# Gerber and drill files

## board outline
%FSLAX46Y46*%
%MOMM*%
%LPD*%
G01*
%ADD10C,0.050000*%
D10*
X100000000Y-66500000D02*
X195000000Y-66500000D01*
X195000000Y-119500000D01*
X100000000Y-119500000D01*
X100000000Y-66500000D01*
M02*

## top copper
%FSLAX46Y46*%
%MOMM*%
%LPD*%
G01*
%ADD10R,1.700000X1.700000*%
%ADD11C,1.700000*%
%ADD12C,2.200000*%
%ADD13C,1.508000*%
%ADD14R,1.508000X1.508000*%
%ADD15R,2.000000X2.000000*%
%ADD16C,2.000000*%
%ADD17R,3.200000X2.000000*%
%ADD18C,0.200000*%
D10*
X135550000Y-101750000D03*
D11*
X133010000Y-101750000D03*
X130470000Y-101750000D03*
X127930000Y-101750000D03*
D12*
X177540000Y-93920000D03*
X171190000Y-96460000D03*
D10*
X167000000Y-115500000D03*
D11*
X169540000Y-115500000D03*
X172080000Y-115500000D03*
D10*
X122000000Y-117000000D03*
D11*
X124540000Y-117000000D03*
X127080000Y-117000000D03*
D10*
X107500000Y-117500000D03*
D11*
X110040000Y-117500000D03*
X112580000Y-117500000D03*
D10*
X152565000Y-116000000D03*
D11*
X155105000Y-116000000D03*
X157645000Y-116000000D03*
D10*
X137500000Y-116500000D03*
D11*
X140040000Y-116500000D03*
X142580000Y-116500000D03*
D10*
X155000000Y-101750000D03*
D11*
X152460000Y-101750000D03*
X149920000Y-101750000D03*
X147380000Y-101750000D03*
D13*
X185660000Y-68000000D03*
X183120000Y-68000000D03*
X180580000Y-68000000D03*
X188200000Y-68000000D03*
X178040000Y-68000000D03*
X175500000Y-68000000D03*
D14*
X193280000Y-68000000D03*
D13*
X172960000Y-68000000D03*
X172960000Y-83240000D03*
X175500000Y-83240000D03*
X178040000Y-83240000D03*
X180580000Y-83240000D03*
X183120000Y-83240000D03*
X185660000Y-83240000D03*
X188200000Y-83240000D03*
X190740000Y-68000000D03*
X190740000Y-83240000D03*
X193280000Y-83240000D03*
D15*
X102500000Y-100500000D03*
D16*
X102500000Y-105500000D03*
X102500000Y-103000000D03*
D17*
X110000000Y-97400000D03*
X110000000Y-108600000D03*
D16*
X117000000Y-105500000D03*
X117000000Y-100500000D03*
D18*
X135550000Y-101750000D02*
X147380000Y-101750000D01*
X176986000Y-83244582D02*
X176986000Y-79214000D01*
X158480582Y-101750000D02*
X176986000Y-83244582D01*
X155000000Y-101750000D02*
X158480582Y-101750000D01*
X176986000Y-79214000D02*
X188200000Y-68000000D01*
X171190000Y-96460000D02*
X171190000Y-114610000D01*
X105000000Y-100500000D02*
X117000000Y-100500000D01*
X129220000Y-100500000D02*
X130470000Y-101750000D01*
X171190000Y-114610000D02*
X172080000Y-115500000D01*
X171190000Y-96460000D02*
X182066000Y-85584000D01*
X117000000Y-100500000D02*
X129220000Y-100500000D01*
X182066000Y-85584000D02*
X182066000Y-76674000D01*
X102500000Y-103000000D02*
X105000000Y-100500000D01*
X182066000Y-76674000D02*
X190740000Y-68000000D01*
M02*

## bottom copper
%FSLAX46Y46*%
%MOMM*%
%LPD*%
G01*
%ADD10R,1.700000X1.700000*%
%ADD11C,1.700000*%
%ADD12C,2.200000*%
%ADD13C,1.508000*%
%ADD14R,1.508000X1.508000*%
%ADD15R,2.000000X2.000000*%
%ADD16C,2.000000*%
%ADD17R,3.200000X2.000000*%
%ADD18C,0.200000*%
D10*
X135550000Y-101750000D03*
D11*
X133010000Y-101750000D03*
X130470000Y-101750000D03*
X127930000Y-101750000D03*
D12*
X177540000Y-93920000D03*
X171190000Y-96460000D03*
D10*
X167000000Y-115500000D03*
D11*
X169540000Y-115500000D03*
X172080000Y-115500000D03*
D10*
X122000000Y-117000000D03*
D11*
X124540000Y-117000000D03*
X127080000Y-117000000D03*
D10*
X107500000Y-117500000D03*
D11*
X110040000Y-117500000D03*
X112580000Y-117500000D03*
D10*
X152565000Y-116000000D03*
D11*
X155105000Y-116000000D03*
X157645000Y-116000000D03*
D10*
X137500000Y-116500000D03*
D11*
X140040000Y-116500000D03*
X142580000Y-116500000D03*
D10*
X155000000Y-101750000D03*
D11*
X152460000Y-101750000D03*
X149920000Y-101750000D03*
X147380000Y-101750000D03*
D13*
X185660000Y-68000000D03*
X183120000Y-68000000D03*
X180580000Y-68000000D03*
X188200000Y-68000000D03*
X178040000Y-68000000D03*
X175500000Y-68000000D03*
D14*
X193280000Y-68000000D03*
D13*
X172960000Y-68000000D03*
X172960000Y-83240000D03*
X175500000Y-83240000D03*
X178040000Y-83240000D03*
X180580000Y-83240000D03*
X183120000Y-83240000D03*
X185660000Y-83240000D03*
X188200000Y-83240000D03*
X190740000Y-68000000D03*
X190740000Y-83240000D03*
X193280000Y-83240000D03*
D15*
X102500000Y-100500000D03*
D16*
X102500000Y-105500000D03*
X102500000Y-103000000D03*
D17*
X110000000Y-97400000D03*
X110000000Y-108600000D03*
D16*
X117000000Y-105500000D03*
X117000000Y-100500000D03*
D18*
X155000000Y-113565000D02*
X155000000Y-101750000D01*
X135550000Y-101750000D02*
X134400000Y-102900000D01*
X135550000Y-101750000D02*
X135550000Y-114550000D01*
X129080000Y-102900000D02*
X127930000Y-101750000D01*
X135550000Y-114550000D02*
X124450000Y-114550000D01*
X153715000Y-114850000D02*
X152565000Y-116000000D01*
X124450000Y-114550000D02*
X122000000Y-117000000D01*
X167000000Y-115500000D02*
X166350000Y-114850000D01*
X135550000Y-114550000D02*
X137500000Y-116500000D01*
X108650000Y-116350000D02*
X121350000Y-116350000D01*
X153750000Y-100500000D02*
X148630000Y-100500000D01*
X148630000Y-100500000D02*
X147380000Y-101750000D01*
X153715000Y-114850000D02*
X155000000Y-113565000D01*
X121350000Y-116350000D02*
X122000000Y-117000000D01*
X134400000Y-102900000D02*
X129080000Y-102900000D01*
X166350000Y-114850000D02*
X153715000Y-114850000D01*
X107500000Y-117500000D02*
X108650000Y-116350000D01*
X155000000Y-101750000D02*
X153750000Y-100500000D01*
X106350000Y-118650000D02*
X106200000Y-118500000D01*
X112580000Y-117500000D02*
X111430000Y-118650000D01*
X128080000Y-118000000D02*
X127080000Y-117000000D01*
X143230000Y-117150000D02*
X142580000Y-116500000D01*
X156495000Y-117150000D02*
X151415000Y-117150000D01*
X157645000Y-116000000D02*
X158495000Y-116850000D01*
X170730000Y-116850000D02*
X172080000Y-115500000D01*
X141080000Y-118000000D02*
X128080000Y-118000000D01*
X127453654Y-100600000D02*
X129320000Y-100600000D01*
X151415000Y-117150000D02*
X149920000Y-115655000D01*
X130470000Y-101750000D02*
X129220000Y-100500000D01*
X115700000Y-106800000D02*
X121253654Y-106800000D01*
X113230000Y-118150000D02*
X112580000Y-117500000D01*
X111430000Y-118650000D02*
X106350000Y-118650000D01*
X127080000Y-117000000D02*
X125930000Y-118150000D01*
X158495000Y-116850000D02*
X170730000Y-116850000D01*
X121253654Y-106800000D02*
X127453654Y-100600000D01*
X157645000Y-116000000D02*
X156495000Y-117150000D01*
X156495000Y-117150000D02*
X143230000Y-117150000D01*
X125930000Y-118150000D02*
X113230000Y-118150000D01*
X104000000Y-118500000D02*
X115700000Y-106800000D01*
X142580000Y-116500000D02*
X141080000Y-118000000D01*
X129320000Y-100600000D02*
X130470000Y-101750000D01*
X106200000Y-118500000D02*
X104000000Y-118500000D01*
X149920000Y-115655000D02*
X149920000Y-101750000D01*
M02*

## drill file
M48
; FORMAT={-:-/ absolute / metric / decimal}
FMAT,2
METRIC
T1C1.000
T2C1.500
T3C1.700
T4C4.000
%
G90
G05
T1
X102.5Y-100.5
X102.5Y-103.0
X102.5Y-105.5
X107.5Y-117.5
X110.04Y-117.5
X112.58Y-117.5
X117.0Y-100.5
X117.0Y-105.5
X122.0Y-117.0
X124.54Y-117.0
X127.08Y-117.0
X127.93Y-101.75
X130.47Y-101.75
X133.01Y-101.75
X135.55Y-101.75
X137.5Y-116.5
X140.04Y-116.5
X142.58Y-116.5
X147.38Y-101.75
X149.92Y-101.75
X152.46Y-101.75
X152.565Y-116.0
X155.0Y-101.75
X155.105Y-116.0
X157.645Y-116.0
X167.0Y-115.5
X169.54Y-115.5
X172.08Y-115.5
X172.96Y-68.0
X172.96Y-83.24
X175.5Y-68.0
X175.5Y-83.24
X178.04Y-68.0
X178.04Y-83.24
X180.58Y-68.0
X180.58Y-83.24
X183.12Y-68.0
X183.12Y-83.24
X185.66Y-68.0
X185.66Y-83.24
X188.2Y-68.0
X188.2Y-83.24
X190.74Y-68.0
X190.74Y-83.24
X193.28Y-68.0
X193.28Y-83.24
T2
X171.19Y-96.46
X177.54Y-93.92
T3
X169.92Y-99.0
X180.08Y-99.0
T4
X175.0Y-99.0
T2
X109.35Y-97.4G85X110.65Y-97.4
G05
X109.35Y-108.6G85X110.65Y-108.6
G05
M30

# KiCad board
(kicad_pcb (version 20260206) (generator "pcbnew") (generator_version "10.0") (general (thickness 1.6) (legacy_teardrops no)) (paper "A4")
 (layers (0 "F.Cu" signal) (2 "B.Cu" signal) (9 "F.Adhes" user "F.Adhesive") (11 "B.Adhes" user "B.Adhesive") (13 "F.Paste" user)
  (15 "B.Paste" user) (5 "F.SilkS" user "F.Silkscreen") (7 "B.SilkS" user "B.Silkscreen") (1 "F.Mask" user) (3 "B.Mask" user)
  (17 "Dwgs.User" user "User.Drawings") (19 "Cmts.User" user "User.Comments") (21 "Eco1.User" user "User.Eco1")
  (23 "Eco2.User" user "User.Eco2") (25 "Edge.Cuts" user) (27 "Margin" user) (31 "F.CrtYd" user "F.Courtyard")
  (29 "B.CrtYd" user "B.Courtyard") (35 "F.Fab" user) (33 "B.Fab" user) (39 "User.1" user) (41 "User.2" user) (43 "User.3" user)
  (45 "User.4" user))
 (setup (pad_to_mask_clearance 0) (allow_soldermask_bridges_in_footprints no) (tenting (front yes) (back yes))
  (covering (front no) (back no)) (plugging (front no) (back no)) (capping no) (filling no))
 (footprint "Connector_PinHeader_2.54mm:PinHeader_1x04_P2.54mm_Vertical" (layer "F.Cu") (at 135.55 101.75 -90)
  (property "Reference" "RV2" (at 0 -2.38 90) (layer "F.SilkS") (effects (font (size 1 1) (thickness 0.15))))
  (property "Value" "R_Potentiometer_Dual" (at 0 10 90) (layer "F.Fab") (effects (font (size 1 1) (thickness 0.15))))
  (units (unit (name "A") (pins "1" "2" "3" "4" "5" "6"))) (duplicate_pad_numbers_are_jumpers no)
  (pad "1" thru_hole rect (at 0 0 270) (size 1.7 1.7) (drill 1) (layers "*.Cu" "*.Mask") (remove_unused_layers no) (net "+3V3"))
  (pad "2" thru_hole circle (at 0 2.54 270) (size 1.7 1.7) (drill 1) (layers "*.Cu" "*.Mask") (remove_unused_layers no) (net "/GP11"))
  (pad "3" thru_hole circle (at 0 5.08 270) (size 1.7 1.7) (drill 1) (layers "*.Cu" "*.Mask") (remove_unused_layers no) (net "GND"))
  (pad "4" thru_hole circle (at 0 7.62 270) (size 1.7 1.7) (drill 1) (layers "*.Cu" "*.Mask") (remove_unused_layers no) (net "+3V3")))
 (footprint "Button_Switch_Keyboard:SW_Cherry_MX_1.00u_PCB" (layer "F.Cu") (at 177.54 93.92)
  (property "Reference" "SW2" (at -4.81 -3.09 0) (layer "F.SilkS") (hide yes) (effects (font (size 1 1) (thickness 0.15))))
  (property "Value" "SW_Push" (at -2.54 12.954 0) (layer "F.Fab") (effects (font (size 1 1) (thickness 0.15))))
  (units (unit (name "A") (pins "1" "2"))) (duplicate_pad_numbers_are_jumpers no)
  (pad "" np_thru_hole circle (at -7.62 5.08) (size 1.7 1.7) (drill 1.7) (layers "*.Cu" "*.Mask"))
  (pad "" np_thru_hole circle (at -2.54 5.08) (size 4 4) (drill 4) (layers "*.Cu" "*.Mask"))
  (pad "" np_thru_hole circle (at 2.54 5.08) (size 1.7 1.7) (drill 1.7) (layers "*.Cu" "*.Mask"))
  (pad "1" thru_hole circle (at 0 0) (size 2.2 2.2) (drill 1.5) (layers "*.Cu" "*.Mask") (remove_unused_layers no) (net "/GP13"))
  (pad "2" thru_hole circle (at -6.35 2.54) (size 2.2 2.2) (drill 1.5) (layers "*.Cu" "*.Mask") (remove_unused_layers no) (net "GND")))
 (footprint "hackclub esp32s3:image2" (layer "F.Cu") (at 152.5 79.5)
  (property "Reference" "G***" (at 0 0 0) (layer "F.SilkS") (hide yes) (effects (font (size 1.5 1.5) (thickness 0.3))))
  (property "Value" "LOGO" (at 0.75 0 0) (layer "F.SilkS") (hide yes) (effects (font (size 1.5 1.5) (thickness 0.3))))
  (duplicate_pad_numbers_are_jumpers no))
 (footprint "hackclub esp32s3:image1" (layer "F.Cu") (at 113.5 75.5)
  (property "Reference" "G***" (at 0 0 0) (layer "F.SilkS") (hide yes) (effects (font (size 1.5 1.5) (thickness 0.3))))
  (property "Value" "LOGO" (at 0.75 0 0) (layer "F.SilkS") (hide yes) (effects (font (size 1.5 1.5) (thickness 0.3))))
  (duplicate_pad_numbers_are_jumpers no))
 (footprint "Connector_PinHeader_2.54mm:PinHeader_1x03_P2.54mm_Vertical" (layer "F.Cu") (at 167 115.5 90)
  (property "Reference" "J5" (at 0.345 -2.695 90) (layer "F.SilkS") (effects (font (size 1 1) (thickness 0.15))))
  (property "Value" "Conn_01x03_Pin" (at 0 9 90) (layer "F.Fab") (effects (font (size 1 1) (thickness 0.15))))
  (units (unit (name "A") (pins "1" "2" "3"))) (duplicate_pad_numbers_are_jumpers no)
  (pad "1" thru_hole rect (at 0 0 90) (size 1.7 1.7) (drill 1) (layers "*.Cu" "*.Mask") (remove_unused_layers no) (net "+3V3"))
  (pad "2" thru_hole circle (at 0 2.54 90) (size 1.7 1.7) (drill 1) (layers "*.Cu" "*.Mask") (remove_unused_layers no) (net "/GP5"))
  (pad "3" thru_hole circle (at 0 5.08 90) (size 1.7 1.7) (drill 1) (layers "*.Cu" "*.Mask") (remove_unused_layers no) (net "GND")))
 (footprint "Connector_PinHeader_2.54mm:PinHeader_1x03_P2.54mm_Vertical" (layer "F.Cu") (at 122 117 90)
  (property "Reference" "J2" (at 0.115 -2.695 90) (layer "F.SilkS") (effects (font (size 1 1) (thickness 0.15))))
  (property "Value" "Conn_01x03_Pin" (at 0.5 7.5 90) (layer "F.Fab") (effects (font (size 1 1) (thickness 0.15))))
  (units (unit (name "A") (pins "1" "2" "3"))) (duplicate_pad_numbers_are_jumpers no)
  (pad "1" thru_hole rect (at 0 0 90) (size 1.7 1.7) (drill 1) (layers "*.Cu" "*.Mask") (remove_unused_layers no) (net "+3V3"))
  (pad "2" thru_hole circle (at 0 2.54 90) (size 1.7 1.7) (drill 1) (layers "*.Cu" "*.Mask") (remove_unused_layers no) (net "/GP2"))
  (pad "3" thru_hole circle (at 0 5.08 90) (size 1.7 1.7) (drill 1) (layers "*.Cu" "*.Mask") (remove_unused_layers no) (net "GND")))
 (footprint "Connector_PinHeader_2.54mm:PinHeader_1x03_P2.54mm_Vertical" (layer "F.Cu") (at 107.5 117.5 90)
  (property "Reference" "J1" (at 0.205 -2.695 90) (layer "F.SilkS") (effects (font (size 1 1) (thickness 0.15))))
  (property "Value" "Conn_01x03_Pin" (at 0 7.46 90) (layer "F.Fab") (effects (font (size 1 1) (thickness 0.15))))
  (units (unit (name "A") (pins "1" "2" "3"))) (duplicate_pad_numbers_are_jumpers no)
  (pad "1" thru_hole rect (at 0 0 90) (size 1.7 1.7) (drill 1) (layers "*.Cu" "*.Mask") (remove_unused_layers no) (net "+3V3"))
  (pad "2" thru_hole circle (at 0 2.54 90) (size 1.7 1.7) (drill 1) (layers "*.Cu" "*.Mask") (remove_unused_layers no) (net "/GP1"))
  (pad "3" thru_hole circle (at 0 5.08 90) (size 1.7 1.7) (drill 1) (layers "*.Cu" "*.Mask") (remove_unused_layers no) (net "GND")))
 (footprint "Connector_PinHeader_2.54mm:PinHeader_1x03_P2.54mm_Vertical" (layer "F.Cu") (at 152.565 116 90)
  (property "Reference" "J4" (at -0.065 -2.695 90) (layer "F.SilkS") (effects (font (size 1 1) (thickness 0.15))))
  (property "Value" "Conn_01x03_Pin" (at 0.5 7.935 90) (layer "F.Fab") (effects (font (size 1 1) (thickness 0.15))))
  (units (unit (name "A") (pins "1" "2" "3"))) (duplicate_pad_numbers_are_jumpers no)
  (pad "1" thru_hole rect (at 0 0 90) (size 1.7 1.7) (drill 1) (layers "*.Cu" "*.Mask") (remove_unused_layers no) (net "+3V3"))
  (pad "2" thru_hole circle (at 0 2.54 90) (size 1.7 1.7) (drill 1) (layers "*.Cu" "*.Mask") (remove_unused_layers no) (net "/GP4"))
  (pad "3" thru_hole circle (at 0 5.08 90) (size 1.7 1.7) (drill 1) (layers "*.Cu" "*.Mask") (remove_unused_layers no) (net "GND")))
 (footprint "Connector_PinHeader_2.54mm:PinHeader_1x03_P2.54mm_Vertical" (layer "F.Cu") (at 137.5 116.5 90)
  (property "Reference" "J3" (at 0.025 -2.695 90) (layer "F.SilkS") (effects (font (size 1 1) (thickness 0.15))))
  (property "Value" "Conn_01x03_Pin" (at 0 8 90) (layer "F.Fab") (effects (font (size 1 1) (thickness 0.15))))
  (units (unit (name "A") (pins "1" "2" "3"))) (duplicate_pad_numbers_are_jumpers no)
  (pad "1" thru_hole rect (at 0 0 90) (size 1.7 1.7) (drill 1) (layers "*.Cu" "*.Mask") (remove_unused_layers no) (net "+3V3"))
  (pad "2" thru_hole circle (at 0 2.54 90) (size 1.7 1.7) (drill 1) (layers "*.Cu" "*.Mask") (remove_unused_layers no) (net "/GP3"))
  (pad "3" thru_hole circle (at 0 5.08 90) (size 1.7 1.7) (drill 1) (layers "*.Cu" "*.Mask") (remove_unused_layers no) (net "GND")))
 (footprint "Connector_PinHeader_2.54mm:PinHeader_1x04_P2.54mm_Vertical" (layer "F.Cu") (at 155 101.75 -90)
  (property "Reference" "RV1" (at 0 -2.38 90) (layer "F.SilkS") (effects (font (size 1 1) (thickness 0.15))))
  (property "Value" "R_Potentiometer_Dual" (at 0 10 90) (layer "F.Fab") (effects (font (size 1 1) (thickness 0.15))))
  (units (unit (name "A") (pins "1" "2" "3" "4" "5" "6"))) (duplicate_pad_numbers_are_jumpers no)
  (pad "1" thru_hole rect (at 0 0 270) (size 1.7 1.7) (drill 1) (layers "*.Cu" "*.Mask") (remove_unused_layers no) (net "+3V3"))
  (pad "2" thru_hole circle (at 0 2.54 270) (size 1.7 1.7) (drill 1) (layers "*.Cu" "*.Mask") (remove_unused_layers no) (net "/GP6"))
  (pad "3" thru_hole circle (at 0 5.08 270) (size 1.7 1.7) (drill 1) (layers "*.Cu" "*.Mask") (remove_unused_layers no) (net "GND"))
  (pad "4" thru_hole circle (at 0 7.62 270) (size 1.7 1.7) (drill 1) (layers "*.Cu" "*.Mask") (remove_unused_layers no) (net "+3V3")))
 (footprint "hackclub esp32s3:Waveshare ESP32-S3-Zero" (layer "F.Cu") (at 183.12 75.62 -90)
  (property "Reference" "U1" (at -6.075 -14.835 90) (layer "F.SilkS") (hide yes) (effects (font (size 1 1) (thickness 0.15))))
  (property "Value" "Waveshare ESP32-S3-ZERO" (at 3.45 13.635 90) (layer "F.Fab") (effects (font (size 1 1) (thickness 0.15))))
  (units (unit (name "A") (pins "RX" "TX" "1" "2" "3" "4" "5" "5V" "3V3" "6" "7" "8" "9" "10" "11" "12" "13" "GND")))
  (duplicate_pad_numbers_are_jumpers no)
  (pad "1" thru_hole circle (at -7.62 -2.54 270) (size 1.508 1.508) (drill 1) (layers "*.Cu" "*.Mask") (remove_unused_layers no)
   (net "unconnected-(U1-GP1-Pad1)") (solder_mask_margin 0.102))
  (pad "2" thru_hole circle (at -7.62 0 270) (size 1.508 1.508) (drill 1) (layers "*.Cu" "*.Mask") (remove_unused_layers no)
   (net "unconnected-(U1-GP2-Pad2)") (solder_mask_margin 0.102))
  (pad "3" thru_hole circle (at -7.62 2.54 270) (size 1.508 1.508) (drill 1) (layers "*.Cu" "*.Mask") (remove_unused_layers no)
   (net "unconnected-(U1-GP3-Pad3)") (solder_mask_margin 0.102))
  (pad "3V3" thru_hole circle (at -7.62 -5.08 270) (size 1.508 1.508) (drill 1) (layers "*.Cu" "*.Mask") (remove_unused_layers no)
   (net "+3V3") (solder_mask_margin 0.102))
  (pad "4" thru_hole circle (at -7.62 5.08 270) (size 1.508 1.508) (drill 1) (layers "*.Cu" "*.Mask") (remove_unused_layers no)
   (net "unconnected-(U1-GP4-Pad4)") (solder_mask_margin 0.102))
  (pad "5" thru_hole circle (at -7.62 7.62 270) (size 1.508 1.508) (drill 1) (layers "*.Cu" "*.Mask") (remove_unused_layers no)
   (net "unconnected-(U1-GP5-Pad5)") (solder_mask_margin 0.102))
  (pad "5V" thru_hole rect (at -7.62 -10.16 270) (size 1.508 1.508) (drill 1) (layers "*.Cu" "*.Mask") (remove_unused_layers no) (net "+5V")
   (solder_mask_margin 0.102))
  (pad "6" thru_hole circle (at -7.62 10.16 270) (size 1.508 1.508) (drill 1) (layers "*.Cu" "*.Mask") (remove_unused_layers no)
   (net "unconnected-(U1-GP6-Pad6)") (solder_mask_margin 0.102))
  (pad "7" thru_hole circle (at 7.62 10.16 270) (size 1.508 1.508) (drill 1) (layers "*.Cu" "*.Mask") (remove_unused_layers no)
   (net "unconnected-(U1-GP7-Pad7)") (solder_mask_margin 0.102))
  (pad "8" thru_hole circle (at 7.62 7.62 270) (size 1.508 1.508) (drill 1) (layers "*.Cu" "*.Mask") (remove_unused_layers no)
   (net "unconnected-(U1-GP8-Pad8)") (solder_mask_margin 0.102))
  (pad "9" thru_hole circle (at 7.62 5.08 270) (size 1.508 1.508) (drill 1) (layers "*.Cu" "*.Mask") (remove_unused_layers no)
   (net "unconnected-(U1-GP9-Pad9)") (solder_mask_margin 0.102))
  (pad "10" thru_hole circle (at 7.62 2.54 270) (size 1.508 1.508) (drill 1) (layers "*.Cu" "*.Mask") (remove_unused_layers no)
   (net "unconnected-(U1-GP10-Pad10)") (solder_mask_margin 0.102))
  (pad "11" thru_hole circle (at 7.62 0 270) (size 1.508 1.508) (drill 1) (layers "*.Cu" "*.Mask") (remove_unused_layers no)
   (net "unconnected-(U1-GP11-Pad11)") (solder_mask_margin 0.102))
  (pad "12" thru_hole circle (at 7.62 -2.54 270) (size 1.508 1.508) (drill 1) (layers "*.Cu" "*.Mask") (remove_unused_layers no)
   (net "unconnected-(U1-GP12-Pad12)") (solder_mask_margin 0.102))
  (pad "13" thru_hole circle (at 7.62 -5.08 270) (size 1.508 1.508) (drill 1) (layers "*.Cu" "*.Mask") (remove_unused_layers no)
   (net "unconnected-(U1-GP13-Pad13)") (solder_mask_margin 0.102))
  (pad "GND" thru_hole circle (at -7.62 -7.62 270) (size 1.508 1.508) (drill 1) (layers "*.Cu" "*.Mask") (remove_unused_layers no)
   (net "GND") (solder_mask_margin 0.102))
  (pad "RX" thru_hole circle (at 7.62 -7.62 270) (size 1.508 1.508) (drill 1) (layers "*.Cu" "*.Mask") (remove_unused_layers no)
   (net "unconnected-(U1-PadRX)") (solder_mask_margin 0.102))
  (pad "TX" thru_hole circle (at 7.62 -10.16 270) (size 1.508 1.508) (drill 1) (layers "*.Cu" "*.Mask") (remove_unused_layers no)
   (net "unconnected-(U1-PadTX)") (solder_mask_margin 0.102)))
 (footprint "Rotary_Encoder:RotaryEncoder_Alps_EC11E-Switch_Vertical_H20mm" (layer "F.Cu") (at 102.5 100.5)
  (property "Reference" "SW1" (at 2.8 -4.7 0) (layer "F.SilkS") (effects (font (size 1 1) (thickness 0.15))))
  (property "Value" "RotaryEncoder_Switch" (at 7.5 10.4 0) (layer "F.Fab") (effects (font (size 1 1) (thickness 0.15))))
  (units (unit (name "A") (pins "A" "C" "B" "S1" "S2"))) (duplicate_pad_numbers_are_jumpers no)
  (pad "A" thru_hole rect (at 0 0) (size 2 2) (drill 1) (layers "*.Cu" "*.Mask") (remove_unused_layers no) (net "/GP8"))
  (pad "B" thru_hole circle (at 0 5) (size 2 2) (drill 1) (layers "*.Cu" "*.Mask") (remove_unused_layers no) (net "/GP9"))
  (pad "C" thru_hole circle (at 0 2.5) (size 2 2) (drill 1) (layers "*.Cu" "*.Mask") (remove_unused_layers no) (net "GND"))
  (pad "MP" thru_hole rect (at 7.5 -3.1) (size 3.2 2) (drill oval 2.8 1.5) (layers "*.Cu" "*.Mask") (remove_unused_layers no))
  (pad "MP" thru_hole rect (at 7.5 8.1) (size 3.2 2) (drill oval 2.8 1.5) (layers "*.Cu" "*.Mask") (remove_unused_layers no))
  (pad "S1" thru_hole circle (at 14.5 5) (size 2 2) (drill 1) (layers "*.Cu" "*.Mask") (remove_unused_layers no) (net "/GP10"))
  (pad "S2" thru_hole circle (at 14.5 0) (size 2 2) (drill 1) (layers "*.Cu" "*.Mask") (remove_unused_layers no) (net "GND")))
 (gr_rect (start 100 66.5) (end 195 119.5) (stroke (width 0.05) (type default)) (fill no) (layer "Edge.Cuts"))
 (segment (start 135.55 101.75) (end 147.38 101.75) (width 0.2) (layer "F.Cu") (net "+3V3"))
 (segment (start 176.986 83.244582) (end 176.986 79.214) (width 0.2) (layer "F.Cu") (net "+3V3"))
 (segment (start 158.480582 101.75) (end 176.986 83.244582) (width 0.2) (layer "F.Cu") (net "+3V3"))
 (segment (start 155 101.75) (end 158.480582 101.75) (width 0.2) (layer "F.Cu") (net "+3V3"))
 (segment (start 176.986 79.214) (end 188.2 68) (width 0.2) (layer "F.Cu") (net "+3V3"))
 (segment (start 155 113.565) (end 155 101.75) (width 0.2) (layer "B.Cu") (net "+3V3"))
 (segment (start 135.55 101.75) (end 134.4 102.9) (width 0.2) (layer "B.Cu") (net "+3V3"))
 (segment (start 135.55 101.75) (end 135.55 114.55) (width 0.2) (layer "B.Cu") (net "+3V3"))
 (segment (start 129.08 102.9) (end 127.93 101.75) (width 0.2) (layer "B.Cu") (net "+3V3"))
 (segment (start 135.55 114.55) (end 124.45 114.55) (width 0.2) (layer "B.Cu") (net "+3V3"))
 (segment (start 153.715 114.85) (end 152.565 116) (width 0.2) (layer "B.Cu") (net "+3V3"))
 (segment (start 124.45 114.55) (end 122 117) (width 0.2) (layer "B.Cu") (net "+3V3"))
 (segment (start 167 115.5) (end 166.35 114.85) (width 0.2) (layer "B.Cu") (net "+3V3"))
 (segment (start 135.55 114.55) (end 137.5 116.5) (width 0.2) (layer "B.Cu") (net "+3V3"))
 (segment (start 108.65 116.35) (end 121.35 116.35) (width 0.2) (layer "B.Cu") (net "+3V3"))
 (segment (start 153.75 100.5) (end 148.63 100.5) (width 0.2) (layer "B.Cu") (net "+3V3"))
 (segment (start 148.63 100.5) (end 147.38 101.75) (width 0.2) (layer "B.Cu") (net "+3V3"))
 (segment (start 153.715 114.85) (end 155 113.565) (width 0.2) (layer "B.Cu") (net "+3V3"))
 (segment (start 121.35 116.35) (end 122 117) (width 0.2) (layer "B.Cu") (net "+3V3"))
 (segment (start 134.4 102.9) (end 129.08 102.9) (width 0.2) (layer "B.Cu") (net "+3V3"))
 (segment (start 166.35 114.85) (end 153.715 114.85) (width 0.2) (layer "B.Cu") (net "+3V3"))
 (segment (start 107.5 117.5) (end 108.65 116.35) (width 0.2) (layer "B.Cu") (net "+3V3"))
 (segment (start 155 101.75) (end 153.75 100.5) (width 0.2) (layer "B.Cu") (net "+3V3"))
 (segment (start 171.19 96.46) (end 171.19 114.61) (width 0.2) (layer "F.Cu") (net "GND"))
 (segment (start 105 100.5) (end 117 100.5) (width 0.2) (layer "F.Cu") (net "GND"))
 (segment (start 129.22 100.5) (end 130.47 101.75) (width 0.2) (layer "F.Cu") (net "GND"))
 (segment (start 171.19 114.61) (end 172.08 115.5) (width 0.2) (layer "F.Cu") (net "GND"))
 (segment (start 171.19 96.46) (end 182.066 85.584) (width 0.2) (layer "F.Cu") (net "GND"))
 (segment (start 117 100.5) (end 129.22 100.5) (width 0.2) (layer "F.Cu") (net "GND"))
 (segment (start 182.066 85.584) (end 182.066 76.674) (width 0.2) (layer "F.Cu") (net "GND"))
 (segment (start 102.5 103) (end 105 100.5) (width 0.2) (layer "F.Cu") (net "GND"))
 (segment (start 182.066 76.674) (end 190.74 68) (width 0.2) (layer "F.Cu") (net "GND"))
 (segment (start 106.35 118.65) (end 106.2 118.5) (width 0.2) (layer "B.Cu") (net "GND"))
 (segment (start 112.58 117.5) (end 111.43 118.65) (width 0.2) (layer "B.Cu") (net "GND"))
 (segment (start 128.08 118) (end 127.08 117) (width 0.2) (layer "B.Cu") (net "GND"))
 (segment (start 143.23 117.15) (end 142.58 116.5) (width 0.2) (layer "B.Cu") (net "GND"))
 (segment (start 156.495 117.15) (end 151.415 117.15) (width 0.2) (layer "B.Cu") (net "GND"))
 (segment (start 157.645 116) (end 158.495 116.85) (width 0.2) (layer "B.Cu") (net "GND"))
 (segment (start 170.73 116.85) (end 172.08 115.5) (width 0.2) (layer "B.Cu") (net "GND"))
 (segment (start 141.08 118) (end 128.08 118) (width 0.2) (layer "B.Cu") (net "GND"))
 (segment (start 127.453654 100.6) (end 129.32 100.6) (width 0.2) (layer "B.Cu") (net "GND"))
 (segment (start 151.415 117.15) (end 149.92 115.655) (width 0.2) (layer "B.Cu") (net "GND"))
 (segment (start 130.47 101.75) (end 129.22 100.5) (width 0.2) (layer "B.Cu") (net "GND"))
 (segment (start 115.7 106.8) (end 121.253654 106.8) (width 0.2) (layer "B.Cu") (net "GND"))
 (segment (start 113.23 118.15) (end 112.58 117.5) (width 0.2) (layer "B.Cu") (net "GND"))
 (segment (start 111.43 118.65) (end 106.35 118.65) (width 0.2) (layer "B.Cu") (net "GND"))
 (segment (start 127.08 117) (end 125.93 118.15) (width 0.2) (layer "B.Cu") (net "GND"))
 (segment (start 158.495 116.85) (end 170.73 116.85) (width 0.2) (layer "B.Cu") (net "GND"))
 (segment (start 121.253654 106.8) (end 127.453654 100.6) (width 0.2) (layer "B.Cu") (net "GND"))
 (segment (start 157.645 116) (end 156.495 117.15) (width 0.2) (layer "B.Cu") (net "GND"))
 (segment (start 156.495 117.15) (end 143.23 117.15) (width 0.2) (layer "B.Cu") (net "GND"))
 (segment (start 125.93 118.15) (end 113.23 118.15) (width 0.2) (layer "B.Cu") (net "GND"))
 (segment (start 104 118.5) (end 115.7 106.8) (width 0.2) (layer "B.Cu") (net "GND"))
 (segment (start 142.58 116.5) (end 141.08 118) (width 0.2) (layer "B.Cu") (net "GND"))
 (segment (start 129.32 100.6) (end 130.47 101.75) (width 0.2) (layer "B.Cu") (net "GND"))
 (segment (start 106.2 118.5) (end 104 118.5) (width 0.2) (layer "B.Cu") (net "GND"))
 (segment (start 149.92 115.655) (end 149.92 101.75) (width 0.2) (layer "B.Cu") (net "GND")))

